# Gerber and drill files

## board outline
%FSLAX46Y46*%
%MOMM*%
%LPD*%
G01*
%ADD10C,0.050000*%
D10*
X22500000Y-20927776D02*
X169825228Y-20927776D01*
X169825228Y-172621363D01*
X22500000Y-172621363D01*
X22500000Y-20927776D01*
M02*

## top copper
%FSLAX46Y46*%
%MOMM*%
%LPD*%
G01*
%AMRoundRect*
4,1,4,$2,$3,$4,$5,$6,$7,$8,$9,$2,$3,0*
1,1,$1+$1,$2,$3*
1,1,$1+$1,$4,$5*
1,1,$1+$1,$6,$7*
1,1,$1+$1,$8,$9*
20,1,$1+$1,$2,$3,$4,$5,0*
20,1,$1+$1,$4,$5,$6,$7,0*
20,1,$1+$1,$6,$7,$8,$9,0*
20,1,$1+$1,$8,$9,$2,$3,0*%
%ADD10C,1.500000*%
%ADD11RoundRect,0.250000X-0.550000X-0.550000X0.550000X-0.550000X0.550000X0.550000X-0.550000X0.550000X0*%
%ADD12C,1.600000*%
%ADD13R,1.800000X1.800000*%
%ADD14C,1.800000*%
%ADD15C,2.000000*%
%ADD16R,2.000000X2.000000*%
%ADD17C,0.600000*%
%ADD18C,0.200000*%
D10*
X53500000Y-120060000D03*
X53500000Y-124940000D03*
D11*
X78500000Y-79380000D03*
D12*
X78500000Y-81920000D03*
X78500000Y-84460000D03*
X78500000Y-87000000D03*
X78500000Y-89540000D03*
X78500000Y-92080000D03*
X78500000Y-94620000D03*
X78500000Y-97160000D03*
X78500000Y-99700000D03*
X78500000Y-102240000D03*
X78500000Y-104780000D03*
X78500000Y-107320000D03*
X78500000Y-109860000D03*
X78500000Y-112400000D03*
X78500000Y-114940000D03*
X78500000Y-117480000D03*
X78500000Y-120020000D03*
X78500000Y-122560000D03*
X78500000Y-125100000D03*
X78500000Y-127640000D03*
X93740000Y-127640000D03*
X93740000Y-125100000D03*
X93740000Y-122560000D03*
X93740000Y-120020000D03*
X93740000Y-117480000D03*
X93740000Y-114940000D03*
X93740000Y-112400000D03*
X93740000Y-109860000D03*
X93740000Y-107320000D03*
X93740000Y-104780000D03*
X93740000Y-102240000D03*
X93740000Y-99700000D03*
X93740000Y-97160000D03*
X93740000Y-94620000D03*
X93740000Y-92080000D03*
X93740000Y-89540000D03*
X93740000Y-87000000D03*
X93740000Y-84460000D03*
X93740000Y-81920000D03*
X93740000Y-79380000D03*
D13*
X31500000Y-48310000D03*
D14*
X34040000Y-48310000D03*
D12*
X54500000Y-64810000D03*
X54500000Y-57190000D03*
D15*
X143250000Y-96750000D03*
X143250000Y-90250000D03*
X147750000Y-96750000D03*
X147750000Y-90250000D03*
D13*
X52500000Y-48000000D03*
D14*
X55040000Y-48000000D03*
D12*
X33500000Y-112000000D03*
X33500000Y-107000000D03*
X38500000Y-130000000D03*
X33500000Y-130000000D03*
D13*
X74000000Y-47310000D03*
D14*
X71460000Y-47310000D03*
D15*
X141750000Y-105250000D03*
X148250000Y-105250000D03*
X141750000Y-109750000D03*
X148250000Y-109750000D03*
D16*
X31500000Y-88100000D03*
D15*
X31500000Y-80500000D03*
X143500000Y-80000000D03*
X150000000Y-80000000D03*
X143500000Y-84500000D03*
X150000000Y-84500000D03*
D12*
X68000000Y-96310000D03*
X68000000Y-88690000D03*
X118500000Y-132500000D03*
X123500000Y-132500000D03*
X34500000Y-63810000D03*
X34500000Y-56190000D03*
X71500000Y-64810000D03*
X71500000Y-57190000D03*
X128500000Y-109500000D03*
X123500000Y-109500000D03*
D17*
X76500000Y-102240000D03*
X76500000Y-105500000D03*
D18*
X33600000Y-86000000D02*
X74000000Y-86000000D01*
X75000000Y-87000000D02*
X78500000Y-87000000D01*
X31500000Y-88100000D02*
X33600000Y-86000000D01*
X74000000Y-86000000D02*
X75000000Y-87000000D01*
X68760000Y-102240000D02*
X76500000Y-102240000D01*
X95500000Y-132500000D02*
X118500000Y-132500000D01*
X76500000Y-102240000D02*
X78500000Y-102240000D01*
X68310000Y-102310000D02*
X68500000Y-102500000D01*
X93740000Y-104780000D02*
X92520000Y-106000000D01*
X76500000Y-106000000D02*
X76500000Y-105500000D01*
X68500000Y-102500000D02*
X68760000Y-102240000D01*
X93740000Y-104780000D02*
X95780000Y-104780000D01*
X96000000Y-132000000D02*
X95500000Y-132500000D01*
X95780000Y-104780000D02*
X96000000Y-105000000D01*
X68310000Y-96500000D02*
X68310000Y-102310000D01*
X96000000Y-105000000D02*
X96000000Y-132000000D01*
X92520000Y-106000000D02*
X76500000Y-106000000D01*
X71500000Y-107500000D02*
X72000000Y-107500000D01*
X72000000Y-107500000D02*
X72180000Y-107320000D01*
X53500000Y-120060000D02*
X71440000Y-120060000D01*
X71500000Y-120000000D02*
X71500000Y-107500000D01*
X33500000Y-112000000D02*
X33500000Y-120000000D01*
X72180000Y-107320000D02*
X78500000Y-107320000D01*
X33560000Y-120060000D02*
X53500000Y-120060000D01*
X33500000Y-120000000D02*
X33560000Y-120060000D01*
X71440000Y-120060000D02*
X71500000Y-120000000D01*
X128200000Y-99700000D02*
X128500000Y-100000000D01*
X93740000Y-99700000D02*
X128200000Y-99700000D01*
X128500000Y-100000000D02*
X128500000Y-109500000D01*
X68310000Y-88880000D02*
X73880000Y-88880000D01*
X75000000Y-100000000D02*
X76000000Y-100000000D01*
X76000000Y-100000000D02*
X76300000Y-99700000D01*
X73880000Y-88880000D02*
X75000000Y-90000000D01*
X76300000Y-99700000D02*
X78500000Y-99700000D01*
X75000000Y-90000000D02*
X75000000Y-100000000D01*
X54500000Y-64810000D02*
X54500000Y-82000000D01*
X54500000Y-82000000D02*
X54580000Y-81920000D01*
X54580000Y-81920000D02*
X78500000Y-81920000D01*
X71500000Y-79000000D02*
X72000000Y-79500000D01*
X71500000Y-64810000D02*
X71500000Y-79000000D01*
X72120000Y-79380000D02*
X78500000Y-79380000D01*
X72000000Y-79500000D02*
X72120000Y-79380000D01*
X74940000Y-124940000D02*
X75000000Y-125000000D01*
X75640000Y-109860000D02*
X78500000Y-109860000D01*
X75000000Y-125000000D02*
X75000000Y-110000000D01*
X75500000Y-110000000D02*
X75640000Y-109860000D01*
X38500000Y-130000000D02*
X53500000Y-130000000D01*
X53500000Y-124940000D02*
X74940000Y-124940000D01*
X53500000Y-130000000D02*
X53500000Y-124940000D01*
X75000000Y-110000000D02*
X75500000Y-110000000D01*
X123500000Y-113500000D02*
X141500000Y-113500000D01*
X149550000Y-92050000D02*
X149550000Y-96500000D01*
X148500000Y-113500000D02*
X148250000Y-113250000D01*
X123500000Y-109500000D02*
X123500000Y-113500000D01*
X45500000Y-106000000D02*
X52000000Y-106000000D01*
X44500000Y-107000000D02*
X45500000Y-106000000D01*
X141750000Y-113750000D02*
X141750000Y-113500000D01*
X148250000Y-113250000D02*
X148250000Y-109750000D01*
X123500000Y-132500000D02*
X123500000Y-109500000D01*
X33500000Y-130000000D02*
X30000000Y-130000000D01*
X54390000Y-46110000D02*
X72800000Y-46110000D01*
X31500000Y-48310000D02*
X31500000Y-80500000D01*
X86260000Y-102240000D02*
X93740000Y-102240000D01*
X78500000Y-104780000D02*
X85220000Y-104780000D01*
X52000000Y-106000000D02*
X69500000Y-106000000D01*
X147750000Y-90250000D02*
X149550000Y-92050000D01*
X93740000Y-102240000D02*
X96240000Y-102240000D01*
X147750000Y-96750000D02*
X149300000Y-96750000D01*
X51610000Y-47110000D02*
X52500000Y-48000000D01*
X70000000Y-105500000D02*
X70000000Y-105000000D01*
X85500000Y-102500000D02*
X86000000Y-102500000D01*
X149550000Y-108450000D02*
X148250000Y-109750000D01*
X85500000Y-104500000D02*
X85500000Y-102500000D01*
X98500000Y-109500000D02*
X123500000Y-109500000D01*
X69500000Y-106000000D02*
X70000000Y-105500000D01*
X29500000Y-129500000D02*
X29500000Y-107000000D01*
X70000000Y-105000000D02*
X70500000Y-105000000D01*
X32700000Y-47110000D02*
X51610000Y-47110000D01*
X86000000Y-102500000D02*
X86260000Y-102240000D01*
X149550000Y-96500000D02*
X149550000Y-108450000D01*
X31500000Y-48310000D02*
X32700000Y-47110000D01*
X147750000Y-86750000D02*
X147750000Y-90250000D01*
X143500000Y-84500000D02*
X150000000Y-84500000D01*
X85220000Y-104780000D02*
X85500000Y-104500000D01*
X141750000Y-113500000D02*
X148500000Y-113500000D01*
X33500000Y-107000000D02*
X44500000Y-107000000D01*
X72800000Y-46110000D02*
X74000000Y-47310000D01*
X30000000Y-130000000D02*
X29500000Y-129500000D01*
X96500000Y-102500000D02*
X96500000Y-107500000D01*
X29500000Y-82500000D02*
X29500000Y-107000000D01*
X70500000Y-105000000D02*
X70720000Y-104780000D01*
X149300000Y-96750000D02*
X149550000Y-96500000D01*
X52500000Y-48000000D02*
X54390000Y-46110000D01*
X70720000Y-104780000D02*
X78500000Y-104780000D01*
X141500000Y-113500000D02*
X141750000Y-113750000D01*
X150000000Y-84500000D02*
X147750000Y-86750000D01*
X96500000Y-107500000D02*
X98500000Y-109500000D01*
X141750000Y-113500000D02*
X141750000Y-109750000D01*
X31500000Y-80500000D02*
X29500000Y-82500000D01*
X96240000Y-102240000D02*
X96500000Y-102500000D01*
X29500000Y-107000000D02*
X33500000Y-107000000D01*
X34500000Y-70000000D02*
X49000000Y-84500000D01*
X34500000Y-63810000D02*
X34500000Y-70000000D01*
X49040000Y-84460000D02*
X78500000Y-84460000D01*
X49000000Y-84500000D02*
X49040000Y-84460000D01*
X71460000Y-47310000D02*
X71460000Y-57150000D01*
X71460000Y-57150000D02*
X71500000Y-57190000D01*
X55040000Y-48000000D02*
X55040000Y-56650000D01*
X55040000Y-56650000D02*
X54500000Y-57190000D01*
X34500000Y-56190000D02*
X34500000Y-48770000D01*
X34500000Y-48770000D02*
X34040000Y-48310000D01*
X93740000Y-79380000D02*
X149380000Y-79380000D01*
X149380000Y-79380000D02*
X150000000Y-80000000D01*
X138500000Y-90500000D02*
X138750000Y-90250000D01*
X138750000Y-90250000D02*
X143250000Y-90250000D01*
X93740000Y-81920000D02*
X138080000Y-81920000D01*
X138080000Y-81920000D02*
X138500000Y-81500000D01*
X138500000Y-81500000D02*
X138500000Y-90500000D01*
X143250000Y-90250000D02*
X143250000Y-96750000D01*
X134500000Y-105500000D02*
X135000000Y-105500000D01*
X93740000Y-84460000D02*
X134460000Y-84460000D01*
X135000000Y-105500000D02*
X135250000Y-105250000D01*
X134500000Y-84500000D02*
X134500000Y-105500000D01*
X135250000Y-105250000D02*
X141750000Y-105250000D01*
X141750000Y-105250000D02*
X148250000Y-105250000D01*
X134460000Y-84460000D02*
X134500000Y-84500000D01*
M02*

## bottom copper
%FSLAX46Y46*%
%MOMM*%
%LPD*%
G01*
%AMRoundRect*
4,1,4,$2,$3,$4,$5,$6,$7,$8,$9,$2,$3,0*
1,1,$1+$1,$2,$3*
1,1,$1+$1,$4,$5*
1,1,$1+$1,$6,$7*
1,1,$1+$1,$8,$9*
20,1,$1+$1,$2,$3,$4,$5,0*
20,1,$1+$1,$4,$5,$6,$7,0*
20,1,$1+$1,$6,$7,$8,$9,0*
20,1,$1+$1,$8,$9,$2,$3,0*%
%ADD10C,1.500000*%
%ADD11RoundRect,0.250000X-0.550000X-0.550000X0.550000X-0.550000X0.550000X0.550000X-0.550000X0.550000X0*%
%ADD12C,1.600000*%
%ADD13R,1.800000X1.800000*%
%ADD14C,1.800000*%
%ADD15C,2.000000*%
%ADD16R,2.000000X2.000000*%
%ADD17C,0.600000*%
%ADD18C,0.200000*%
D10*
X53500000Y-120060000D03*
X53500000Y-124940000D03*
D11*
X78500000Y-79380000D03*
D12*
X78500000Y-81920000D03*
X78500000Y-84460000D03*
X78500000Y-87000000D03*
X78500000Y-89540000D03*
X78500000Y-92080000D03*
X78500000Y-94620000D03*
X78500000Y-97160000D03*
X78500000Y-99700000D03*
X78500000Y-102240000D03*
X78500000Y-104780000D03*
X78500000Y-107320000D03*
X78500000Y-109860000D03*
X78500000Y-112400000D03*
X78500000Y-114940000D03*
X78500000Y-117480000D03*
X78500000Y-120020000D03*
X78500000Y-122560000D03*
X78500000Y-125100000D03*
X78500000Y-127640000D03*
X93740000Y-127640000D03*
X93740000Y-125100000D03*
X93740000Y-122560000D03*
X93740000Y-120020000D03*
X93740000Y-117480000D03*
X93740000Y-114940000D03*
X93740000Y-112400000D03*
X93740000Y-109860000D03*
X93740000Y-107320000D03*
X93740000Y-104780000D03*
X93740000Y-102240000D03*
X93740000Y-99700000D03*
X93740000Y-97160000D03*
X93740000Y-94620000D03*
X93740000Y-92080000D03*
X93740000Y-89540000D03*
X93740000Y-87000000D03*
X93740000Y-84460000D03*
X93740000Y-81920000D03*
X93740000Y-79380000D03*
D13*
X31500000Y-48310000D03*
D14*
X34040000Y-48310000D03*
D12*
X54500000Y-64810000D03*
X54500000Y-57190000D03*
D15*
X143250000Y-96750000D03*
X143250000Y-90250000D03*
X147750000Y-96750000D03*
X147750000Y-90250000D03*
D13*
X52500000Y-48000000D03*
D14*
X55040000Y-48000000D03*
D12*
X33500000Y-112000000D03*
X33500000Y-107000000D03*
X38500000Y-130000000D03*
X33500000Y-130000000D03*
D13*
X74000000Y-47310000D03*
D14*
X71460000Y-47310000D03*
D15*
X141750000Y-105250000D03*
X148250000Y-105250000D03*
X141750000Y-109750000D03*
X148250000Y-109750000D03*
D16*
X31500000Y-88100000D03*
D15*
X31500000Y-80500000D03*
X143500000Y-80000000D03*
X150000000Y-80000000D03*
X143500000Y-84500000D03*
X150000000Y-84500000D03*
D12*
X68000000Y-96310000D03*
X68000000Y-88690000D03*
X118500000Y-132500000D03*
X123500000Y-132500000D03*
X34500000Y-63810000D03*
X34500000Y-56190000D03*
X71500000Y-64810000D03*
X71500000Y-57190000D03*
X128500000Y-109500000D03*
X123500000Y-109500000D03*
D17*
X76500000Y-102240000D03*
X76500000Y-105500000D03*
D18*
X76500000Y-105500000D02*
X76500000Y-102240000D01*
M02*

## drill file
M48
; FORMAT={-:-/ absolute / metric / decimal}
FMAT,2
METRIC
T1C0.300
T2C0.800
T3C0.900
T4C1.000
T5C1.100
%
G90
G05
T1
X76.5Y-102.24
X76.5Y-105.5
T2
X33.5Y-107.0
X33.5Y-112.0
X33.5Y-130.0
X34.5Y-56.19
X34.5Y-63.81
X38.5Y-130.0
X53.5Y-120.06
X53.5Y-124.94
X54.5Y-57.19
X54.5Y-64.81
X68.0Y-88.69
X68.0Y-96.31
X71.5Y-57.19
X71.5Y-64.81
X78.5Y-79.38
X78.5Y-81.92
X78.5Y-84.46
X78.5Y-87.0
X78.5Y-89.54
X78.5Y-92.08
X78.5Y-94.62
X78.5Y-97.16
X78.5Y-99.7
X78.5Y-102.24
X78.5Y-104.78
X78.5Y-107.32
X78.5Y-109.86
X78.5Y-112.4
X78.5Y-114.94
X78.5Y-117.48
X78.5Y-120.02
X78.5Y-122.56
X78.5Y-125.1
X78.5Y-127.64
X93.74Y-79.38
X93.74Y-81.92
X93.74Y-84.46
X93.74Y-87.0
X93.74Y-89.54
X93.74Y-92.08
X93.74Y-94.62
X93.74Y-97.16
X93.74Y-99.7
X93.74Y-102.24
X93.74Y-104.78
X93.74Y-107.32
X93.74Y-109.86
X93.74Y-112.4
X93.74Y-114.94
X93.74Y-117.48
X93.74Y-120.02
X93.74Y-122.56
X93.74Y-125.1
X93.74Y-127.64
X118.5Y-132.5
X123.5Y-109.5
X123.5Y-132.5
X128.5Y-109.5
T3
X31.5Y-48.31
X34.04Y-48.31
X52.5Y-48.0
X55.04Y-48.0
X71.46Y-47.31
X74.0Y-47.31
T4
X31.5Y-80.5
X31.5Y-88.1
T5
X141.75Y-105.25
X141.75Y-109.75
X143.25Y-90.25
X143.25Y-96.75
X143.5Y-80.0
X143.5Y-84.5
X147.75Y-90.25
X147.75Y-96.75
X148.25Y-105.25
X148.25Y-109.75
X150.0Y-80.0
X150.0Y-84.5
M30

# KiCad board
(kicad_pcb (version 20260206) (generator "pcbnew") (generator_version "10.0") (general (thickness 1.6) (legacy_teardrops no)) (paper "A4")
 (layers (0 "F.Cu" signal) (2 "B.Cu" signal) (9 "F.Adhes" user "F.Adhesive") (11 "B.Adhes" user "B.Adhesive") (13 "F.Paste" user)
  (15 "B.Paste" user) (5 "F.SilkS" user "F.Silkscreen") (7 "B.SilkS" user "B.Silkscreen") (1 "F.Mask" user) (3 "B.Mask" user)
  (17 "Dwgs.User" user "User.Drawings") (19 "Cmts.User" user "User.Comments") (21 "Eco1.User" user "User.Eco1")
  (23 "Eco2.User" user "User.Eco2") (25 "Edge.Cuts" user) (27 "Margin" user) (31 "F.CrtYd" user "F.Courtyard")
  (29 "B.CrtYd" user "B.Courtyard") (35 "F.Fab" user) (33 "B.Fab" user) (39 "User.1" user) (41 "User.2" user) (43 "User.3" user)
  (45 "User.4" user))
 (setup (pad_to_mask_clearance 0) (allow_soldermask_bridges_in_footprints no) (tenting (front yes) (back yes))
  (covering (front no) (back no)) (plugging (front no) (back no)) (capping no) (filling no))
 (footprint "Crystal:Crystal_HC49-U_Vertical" (layer "F.Cu") (at 53.5 120.06 -90)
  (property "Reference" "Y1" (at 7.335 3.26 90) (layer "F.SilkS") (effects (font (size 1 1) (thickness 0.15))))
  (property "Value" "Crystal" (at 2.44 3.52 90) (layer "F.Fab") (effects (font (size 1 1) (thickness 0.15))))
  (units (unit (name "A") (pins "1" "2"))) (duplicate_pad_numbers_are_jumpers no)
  (pad "1" thru_hole circle (at 0 0 270) (size 1.5 1.5) (drill 0.8) (layers "*.Cu" "*.Mask") (remove_unused_layers no)
   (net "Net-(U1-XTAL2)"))
  (pad "2" thru_hole circle (at 4.88 0 270) (size 1.5 1.5) (drill 0.8) (layers "*.Cu" "*.Mask") (remove_unused_layers no)
   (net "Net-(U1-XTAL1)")))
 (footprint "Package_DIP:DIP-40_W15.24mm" (layer "F.Cu") (at 78.5 79.38)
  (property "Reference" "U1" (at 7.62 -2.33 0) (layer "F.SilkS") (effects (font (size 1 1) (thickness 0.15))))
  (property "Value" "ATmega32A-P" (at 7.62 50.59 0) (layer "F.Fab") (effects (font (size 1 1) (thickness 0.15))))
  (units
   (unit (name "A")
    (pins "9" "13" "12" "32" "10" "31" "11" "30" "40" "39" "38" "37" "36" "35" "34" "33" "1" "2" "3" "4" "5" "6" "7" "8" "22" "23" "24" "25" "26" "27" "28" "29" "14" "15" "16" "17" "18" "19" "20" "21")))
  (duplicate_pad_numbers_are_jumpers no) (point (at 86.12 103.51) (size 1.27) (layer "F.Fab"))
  (pad "1" thru_hole roundrect (at 0 0) (size 1.6 1.6) (drill 0.8) (layers "*.Cu" "*.Mask") (remove_unused_layers no)
   (roundrect_rratio 0.15625) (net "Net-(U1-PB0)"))
  (pad "2" thru_hole circle (at 0 2.54) (size 1.6 1.6) (drill 0.8) (layers "*.Cu" "*.Mask") (remove_unused_layers no) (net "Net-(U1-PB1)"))
  (pad "3" thru_hole circle (at 0 5.08) (size 1.6 1.6) (drill 0.8) (layers "*.Cu" "*.Mask") (remove_unused_layers no) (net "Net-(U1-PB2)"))
  (pad "4" thru_hole circle (at 0 7.62) (size 1.6 1.6) (drill 0.8) (layers "*.Cu" "*.Mask") (remove_unused_layers no) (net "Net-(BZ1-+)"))
  (pad "5" thru_hole circle (at 0 10.16) (size 1.6 1.6) (drill 0.8) (layers "*.Cu" "*.Mask") (remove_unused_layers no)
   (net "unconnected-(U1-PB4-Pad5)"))
  (pad "6" thru_hole circle (at 0 12.7) (size 1.6 1.6) (drill 0.8) (layers "*.Cu" "*.Mask") (remove_unused_layers no)
   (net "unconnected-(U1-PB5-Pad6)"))
  (pad "7" thru_hole circle (at 0 15.24) (size 1.6 1.6) (drill 0.8) (layers "*.Cu" "*.Mask") (remove_unused_layers no)
   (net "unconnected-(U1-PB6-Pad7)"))
  (pad "8" thru_hole circle (at 0 17.78) (size 1.6 1.6) (drill 0.8) (layers "*.Cu" "*.Mask") (remove_unused_layers no)
   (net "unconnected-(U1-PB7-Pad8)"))
  (pad "9" thru_hole circle (at 0 20.32) (size 1.6 1.6) (drill 0.8) (layers "*.Cu" "*.Mask") (remove_unused_layers no)
   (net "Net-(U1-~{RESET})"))
  (pad "10" thru_hole circle (at 0 22.86) (size 1.6 1.6) (drill 0.8) (layers "*.Cu" "*.Mask") (remove_unused_layers no) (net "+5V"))
  (pad "11" thru_hole circle (at 0 25.4) (size 1.6 1.6) (drill 0.8) (layers "*.Cu" "*.Mask") (remove_unused_layers no) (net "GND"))
  (pad "12" thru_hole circle (at 0 27.94) (size 1.6 1.6) (drill 0.8) (layers "*.Cu" "*.Mask") (remove_unused_layers no)
   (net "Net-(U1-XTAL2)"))
  (pad "13" thru_hole circle (at 0 30.48) (size 1.6 1.6) (drill 0.8) (layers "*.Cu" "*.Mask") (remove_unused_layers no)
   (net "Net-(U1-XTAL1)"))
  (pad "14" thru_hole circle (at 0 33.02) (size 1.6 1.6) (drill 0.8) (layers "*.Cu" "*.Mask") (remove_unused_layers no)
   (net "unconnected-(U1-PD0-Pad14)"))
  (pad "15" thru_hole circle (at 0 35.56) (size 1.6 1.6) (drill 0.8) (layers "*.Cu" "*.Mask") (remove_unused_layers no)
   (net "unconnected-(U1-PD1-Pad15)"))
  (pad "16" thru_hole circle (at 0 38.1) (size 1.6 1.6) (drill 0.8) (layers "*.Cu" "*.Mask") (remove_unused_layers no)
   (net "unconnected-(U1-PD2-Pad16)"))
  (pad "17" thru_hole circle (at 0 40.64) (size 1.6 1.6) (drill 0.8) (layers "*.Cu" "*.Mask") (remove_unused_layers no)
   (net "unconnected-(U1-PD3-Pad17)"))
  (pad "18" thru_hole circle (at 0 43.18) (size 1.6 1.6) (drill 0.8) (layers "*.Cu" "*.Mask") (remove_unused_layers no)
   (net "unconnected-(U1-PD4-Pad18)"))
  (pad "19" thru_hole circle (at 0 45.72) (size 1.6 1.6) (drill 0.8) (layers "*.Cu" "*.Mask") (remove_unused_layers no)
   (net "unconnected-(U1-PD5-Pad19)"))
  (pad "20" thru_hole circle (at 0 48.26) (size 1.6 1.6) (drill 0.8) (layers "*.Cu" "*.Mask") (remove_unused_layers no)
   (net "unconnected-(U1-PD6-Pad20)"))
  (pad "21" thru_hole circle (at 15.24 48.26) (size 1.6 1.6) (drill 0.8) (layers "*.Cu" "*.Mask") (remove_unused_layers no)
   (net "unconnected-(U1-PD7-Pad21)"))
  (pad "22" thru_hole circle (at 15.24 45.72) (size 1.6 1.6) (drill 0.8) (layers "*.Cu" "*.Mask") (remove_unused_layers no)
   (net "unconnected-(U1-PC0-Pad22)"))
  (pad "23" thru_hole circle (at 15.24 43.18) (size 1.6 1.6) (drill 0.8) (layers "*.Cu" "*.Mask") (remove_unused_layers no)
   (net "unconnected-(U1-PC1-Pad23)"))
  (pad "24" thru_hole circle (at 15.24 40.64) (size 1.6 1.6) (drill 0.8) (layers "*.Cu" "*.Mask") (remove_unused_layers no)
   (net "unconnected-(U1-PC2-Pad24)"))
  (pad "25" thru_hole circle (at 15.24 38.1) (size 1.6 1.6) (drill 0.8) (layers "*.Cu" "*.Mask") (remove_unused_layers no)
   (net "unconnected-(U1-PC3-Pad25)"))
  (pad "26" thru_hole circle (at 15.24 35.56) (size 1.6 1.6) (drill 0.8) (layers "*.Cu" "*.Mask") (remove_unused_layers no)
   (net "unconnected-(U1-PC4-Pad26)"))
  (pad "27" thru_hole circle (at 15.24 33.02) (size 1.6 1.6) (drill 0.8) (layers "*.Cu" "*.Mask") (remove_unused_layers no)
   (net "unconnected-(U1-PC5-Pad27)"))
  (pad "28" thru_hole circle (at 15.24 30.48) (size 1.6 1.6) (drill 0.8) (layers "*.Cu" "*.Mask") (remove_unused_layers no)
   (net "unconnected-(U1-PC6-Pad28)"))
  (pad "29" thru_hole circle (at 15.24 27.94) (size 1.6 1.6) (drill 0.8) (layers "*.Cu" "*.Mask") (remove_unused_layers no)
   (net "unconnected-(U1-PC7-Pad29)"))
  (pad "30" thru_hole circle (at 15.24 25.4) (size 1.6 1.6) (drill 0.8) (layers "*.Cu" "*.Mask") (remove_unused_layers no) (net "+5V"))
  (pad "31" thru_hole circle (at 15.24 22.86) (size 1.6 1.6) (drill 0.8) (layers "*.Cu" "*.Mask") (remove_unused_layers no) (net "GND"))
  (pad "32" thru_hole circle (at 15.24 20.32) (size 1.6 1.6) (drill 0.8) (layers "*.Cu" "*.Mask") (remove_unused_layers no)
   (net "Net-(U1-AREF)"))
  (pad "33" thru_hole circle (at 15.24 17.78) (size 1.6 1.6) (drill 0.8) (layers "*.Cu" "*.Mask") (remove_unused_layers no)
   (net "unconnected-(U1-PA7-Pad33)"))
  (pad "34" thru_hole circle (at 15.24 15.24) (size 1.6 1.6) (drill 0.8) (layers "*.Cu" "*.Mask") (remove_unused_layers no)
   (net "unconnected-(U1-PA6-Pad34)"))
  (pad "35" thru_hole circle (at 15.24 12.7) (size 1.6 1.6) (drill 0.8) (layers "*.Cu" "*.Mask") (remove_unused_layers no)
   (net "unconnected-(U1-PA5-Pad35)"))
  (pad "36" thru_hole circle (at 15.24 10.16) (size 1.6 1.6) (drill 0.8) (layers "*.Cu" "*.Mask") (remove_unused_layers no)
   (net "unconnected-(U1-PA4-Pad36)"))
  (pad "37" thru_hole circle (at 15.24 7.62) (size 1.6 1.6) (drill 0.8) (layers "*.Cu" "*.Mask") (remove_unused_layers no)
   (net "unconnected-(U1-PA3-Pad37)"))
  (pad "38" thru_hole circle (at 15.24 5.08) (size 1.6 1.6) (drill 0.8) (layers "*.Cu" "*.Mask") (remove_unused_layers no)
   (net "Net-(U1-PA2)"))
  (pad "39" thru_hole circle (at 15.24 2.54) (size 1.6 1.6) (drill 0.8) (layers "*.Cu" "*.Mask") (remove_unused_layers no)
   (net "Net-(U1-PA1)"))
  (pad "40" thru_hole circle (at 15.24 0) (size 1.6 1.6) (drill 0.8) (layers "*.Cu" "*.Mask") (remove_unused_layers no) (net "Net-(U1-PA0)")))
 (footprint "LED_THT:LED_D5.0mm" (layer "F.Cu") (at 31.5 48.31)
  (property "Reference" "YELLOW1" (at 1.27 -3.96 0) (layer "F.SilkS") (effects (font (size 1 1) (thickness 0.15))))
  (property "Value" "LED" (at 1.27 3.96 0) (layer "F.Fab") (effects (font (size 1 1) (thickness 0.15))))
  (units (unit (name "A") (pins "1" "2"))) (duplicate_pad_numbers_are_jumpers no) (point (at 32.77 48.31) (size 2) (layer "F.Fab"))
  (pad "1" thru_hole rect (at 0 0) (size 1.8 1.8) (drill 0.9) (layers "*.Cu" "*.Mask") (remove_unused_layers no) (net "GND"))
  (pad "2" thru_hole circle (at 2.54 0) (size 1.8 1.8) (drill 0.9) (layers "*.Cu" "*.Mask") (remove_unused_layers no)
   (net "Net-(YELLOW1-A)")))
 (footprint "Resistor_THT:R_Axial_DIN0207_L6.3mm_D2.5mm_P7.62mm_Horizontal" (layer "F.Cu") (at 54.5 64.81 90)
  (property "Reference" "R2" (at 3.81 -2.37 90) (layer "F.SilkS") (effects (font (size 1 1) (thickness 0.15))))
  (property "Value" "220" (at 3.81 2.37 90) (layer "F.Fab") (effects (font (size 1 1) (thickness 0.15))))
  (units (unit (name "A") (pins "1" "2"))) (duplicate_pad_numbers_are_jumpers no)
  (pad "1" thru_hole circle (at 0 0 90) (size 1.6 1.6) (drill 0.8) (layers "*.Cu" "*.Mask") (remove_unused_layers no) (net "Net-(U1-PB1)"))
  (pad "2" thru_hole circle (at 7.62 0 90) (size 1.6 1.6) (drill 0.8) (layers "*.Cu" "*.Mask") (remove_unused_layers no)
   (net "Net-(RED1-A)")))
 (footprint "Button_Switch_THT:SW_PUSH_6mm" (layer "F.Cu") (at 143.25 96.75 90)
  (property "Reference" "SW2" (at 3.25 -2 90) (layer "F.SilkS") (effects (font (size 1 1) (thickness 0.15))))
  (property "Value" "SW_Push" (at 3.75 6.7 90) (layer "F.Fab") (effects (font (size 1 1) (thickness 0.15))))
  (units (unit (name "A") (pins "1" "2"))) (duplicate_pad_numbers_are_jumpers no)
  (pad "1" thru_hole circle (at 0 0 180) (size 2 2) (drill 1.1) (layers "*.Cu" "*.Mask") (remove_unused_layers no) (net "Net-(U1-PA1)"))
  (pad "1" thru_hole circle (at 6.5 0 180) (size 2 2) (drill 1.1) (layers "*.Cu" "*.Mask") (remove_unused_layers no) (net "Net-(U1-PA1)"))
  (pad "2" thru_hole circle (at 0 4.5 180) (size 2 2) (drill 1.1) (layers "*.Cu" "*.Mask") (remove_unused_layers no) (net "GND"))
  (pad "2" thru_hole circle (at 6.5 4.5 180) (size 2 2) (drill 1.1) (layers "*.Cu" "*.Mask") (remove_unused_layers no) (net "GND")))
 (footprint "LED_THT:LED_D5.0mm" (layer "F.Cu") (at 52.5 48)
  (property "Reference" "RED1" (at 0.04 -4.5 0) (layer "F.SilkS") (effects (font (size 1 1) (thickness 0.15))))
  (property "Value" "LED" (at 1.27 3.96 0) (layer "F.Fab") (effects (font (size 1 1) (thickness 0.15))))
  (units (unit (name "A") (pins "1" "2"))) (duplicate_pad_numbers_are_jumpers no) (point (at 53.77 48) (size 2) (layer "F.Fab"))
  (pad "1" thru_hole rect (at 0 0) (size 1.8 1.8) (drill 0.9) (layers "*.Cu" "*.Mask") (remove_unused_layers no) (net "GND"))
  (pad "2" thru_hole circle (at 2.54 0) (size 1.8 1.8) (drill 0.9) (layers "*.Cu" "*.Mask") (remove_unused_layers no) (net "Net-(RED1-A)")))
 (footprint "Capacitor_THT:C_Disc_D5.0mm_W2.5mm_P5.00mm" (layer "F.Cu") (at 33.5 112 90)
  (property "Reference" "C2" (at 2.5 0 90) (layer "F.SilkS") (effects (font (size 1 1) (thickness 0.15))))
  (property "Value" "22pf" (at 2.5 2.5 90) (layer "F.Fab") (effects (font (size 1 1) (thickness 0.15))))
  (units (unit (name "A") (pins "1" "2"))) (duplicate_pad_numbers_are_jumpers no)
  (pad "1" thru_hole circle (at 0 0 90) (size 1.6 1.6) (drill 0.8) (layers "*.Cu" "*.Mask") (remove_unused_layers no) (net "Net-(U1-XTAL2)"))
  (pad "2" thru_hole circle (at 5 0 90) (size 1.6 1.6) (drill 0.8) (layers "*.Cu" "*.Mask") (remove_unused_layers no) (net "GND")))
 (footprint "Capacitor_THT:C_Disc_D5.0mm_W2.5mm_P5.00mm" (layer "F.Cu") (at 38.5 130 180)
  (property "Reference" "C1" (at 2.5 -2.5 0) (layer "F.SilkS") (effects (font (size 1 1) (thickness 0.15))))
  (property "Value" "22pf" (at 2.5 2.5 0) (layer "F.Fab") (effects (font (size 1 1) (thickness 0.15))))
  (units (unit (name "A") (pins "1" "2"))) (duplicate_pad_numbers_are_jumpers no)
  (pad "1" thru_hole circle (at 0 0 180) (size 1.6 1.6) (drill 0.8) (layers "*.Cu" "*.Mask") (remove_unused_layers no)
   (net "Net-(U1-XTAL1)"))
  (pad "2" thru_hole circle (at 5 0 180) (size 1.6 1.6) (drill 0.8) (layers "*.Cu" "*.Mask") (remove_unused_layers no) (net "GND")))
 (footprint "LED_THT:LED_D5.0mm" (layer "F.Cu") (at 74 47.31 180)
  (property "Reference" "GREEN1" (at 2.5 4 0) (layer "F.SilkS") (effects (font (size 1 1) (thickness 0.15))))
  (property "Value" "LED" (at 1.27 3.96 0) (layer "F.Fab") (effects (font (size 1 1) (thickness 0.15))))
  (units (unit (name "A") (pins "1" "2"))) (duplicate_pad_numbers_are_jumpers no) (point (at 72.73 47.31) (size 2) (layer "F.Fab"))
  (pad "1" thru_hole rect (at 0 0 180) (size 1.8 1.8) (drill 0.9) (layers "*.Cu" "*.Mask") (remove_unused_layers no) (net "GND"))
  (pad "2" thru_hole circle (at 2.54 0 180) (size 1.8 1.8) (drill 0.9) (layers "*.Cu" "*.Mask") (remove_unused_layers no)
   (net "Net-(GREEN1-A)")))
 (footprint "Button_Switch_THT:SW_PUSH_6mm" (layer "F.Cu") (at 141.75 105.25)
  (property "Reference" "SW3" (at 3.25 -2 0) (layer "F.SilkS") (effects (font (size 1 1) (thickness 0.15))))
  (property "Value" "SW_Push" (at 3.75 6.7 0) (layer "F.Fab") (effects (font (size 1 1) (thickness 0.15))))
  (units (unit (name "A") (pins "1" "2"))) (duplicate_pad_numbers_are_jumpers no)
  (pad "1" thru_hole circle (at 0 0 90) (size 2 2) (drill 1.1) (layers "*.Cu" "*.Mask") (remove_unused_layers no) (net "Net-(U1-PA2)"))
  (pad "1" thru_hole circle (at 6.5 0 90) (size 2 2) (drill 1.1) (layers "*.Cu" "*.Mask") (remove_unused_layers no) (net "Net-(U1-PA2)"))
  (pad "2" thru_hole circle (at 0 4.5 90) (size 2 2) (drill 1.1) (layers "*.Cu" "*.Mask") (remove_unused_layers no) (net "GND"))
  (pad "2" thru_hole circle (at 6.5 4.5 90) (size 2 2) (drill 1.1) (layers "*.Cu" "*.Mask") (remove_unused_layers no) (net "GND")))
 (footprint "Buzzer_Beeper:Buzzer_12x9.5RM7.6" (layer "F.Cu") (at 31.5 88.1 90)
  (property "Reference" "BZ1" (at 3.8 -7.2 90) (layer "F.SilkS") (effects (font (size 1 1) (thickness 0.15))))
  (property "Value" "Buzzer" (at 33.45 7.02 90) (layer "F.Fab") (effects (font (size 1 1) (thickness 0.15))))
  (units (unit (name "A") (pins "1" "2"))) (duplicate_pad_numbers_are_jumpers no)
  (pad "1" thru_hole rect (at 0 0 90) (size 2 2) (drill 1) (layers "*.Cu" "*.Mask") (remove_unused_layers no) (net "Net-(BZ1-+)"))
  (pad "2" thru_hole circle (at 7.6 0 90) (size 2 2) (drill 1) (layers "*.Cu" "*.Mask") (remove_unused_layers no) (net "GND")))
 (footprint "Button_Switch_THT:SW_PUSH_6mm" (layer "F.Cu") (at 143.5 80)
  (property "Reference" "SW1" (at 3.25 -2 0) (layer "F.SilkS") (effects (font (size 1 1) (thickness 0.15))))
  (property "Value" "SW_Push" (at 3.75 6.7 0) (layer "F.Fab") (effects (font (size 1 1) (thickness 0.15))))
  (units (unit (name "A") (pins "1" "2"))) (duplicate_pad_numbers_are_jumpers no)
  (pad "1" thru_hole circle (at 0 0 90) (size 2 2) (drill 1.1) (layers "*.Cu" "*.Mask") (remove_unused_layers no) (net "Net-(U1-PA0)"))
  (pad "1" thru_hole circle (at 6.5 0 90) (size 2 2) (drill 1.1) (layers "*.Cu" "*.Mask") (remove_unused_layers no) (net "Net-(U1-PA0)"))
  (pad "2" thru_hole circle (at 0 4.5 90) (size 2 2) (drill 1.1) (layers "*.Cu" "*.Mask") (remove_unused_layers no) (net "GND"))
  (pad "2" thru_hole circle (at 6.5 4.5 90) (size 2 2) (drill 1.1) (layers "*.Cu" "*.Mask") (remove_unused_layers no) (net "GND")))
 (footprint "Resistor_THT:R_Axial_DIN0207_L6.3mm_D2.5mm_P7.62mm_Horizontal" (layer "F.Cu") (at 68 96.31 90)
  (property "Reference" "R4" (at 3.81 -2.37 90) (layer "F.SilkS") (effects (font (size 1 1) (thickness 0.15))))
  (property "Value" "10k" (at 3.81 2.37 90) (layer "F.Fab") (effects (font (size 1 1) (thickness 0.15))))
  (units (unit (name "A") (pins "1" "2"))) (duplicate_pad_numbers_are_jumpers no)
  (pad "1" thru_hole circle (at 0 0 90) (size 1.6 1.6) (drill 0.8) (layers "*.Cu" "*.Mask") (remove_unused_layers no) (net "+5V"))
  (pad "2" thru_hole circle (at 7.62 0 90) (size 1.6 1.6) (drill 0.8) (layers "*.Cu" "*.Mask") (remove_unused_layers no)
   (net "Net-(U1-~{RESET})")))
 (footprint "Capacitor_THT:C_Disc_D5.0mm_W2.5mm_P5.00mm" (layer "F.Cu") (at 118.5 132.5)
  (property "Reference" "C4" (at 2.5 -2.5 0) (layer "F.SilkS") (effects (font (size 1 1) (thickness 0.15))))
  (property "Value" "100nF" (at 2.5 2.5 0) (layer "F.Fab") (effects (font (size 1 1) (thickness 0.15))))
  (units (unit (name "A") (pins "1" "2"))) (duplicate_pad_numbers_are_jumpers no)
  (pad "1" thru_hole circle (at 0 0) (size 1.6 1.6) (drill 0.8) (layers "*.Cu" "*.Mask") (remove_unused_layers no) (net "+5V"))
  (pad "2" thru_hole circle (at 5 0) (size 1.6 1.6) (drill 0.8) (layers "*.Cu" "*.Mask") (remove_unused_layers no) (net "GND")))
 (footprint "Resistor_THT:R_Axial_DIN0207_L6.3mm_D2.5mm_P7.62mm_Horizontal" (layer "F.Cu") (at 34.5 63.81 90)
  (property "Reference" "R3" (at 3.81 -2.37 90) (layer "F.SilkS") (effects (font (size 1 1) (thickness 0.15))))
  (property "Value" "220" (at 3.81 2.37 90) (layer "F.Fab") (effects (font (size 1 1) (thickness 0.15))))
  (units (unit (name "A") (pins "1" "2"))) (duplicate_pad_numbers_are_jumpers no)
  (pad "1" thru_hole circle (at 0 0 90) (size 1.6 1.6) (drill 0.8) (layers "*.Cu" "*.Mask") (remove_unused_layers no) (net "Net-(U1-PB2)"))
  (pad "2" thru_hole circle (at 7.62 0 90) (size 1.6 1.6) (drill 0.8) (layers "*.Cu" "*.Mask") (remove_unused_layers no)
   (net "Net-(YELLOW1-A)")))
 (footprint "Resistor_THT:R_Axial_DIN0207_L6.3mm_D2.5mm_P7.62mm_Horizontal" (layer "F.Cu") (at 71.5 64.81 90)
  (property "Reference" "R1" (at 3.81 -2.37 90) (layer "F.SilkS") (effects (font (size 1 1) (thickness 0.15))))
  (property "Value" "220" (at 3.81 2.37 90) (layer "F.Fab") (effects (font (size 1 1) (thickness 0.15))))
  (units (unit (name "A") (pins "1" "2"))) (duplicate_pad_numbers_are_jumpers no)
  (pad "1" thru_hole circle (at 0 0 90) (size 1.6 1.6) (drill 0.8) (layers "*.Cu" "*.Mask") (remove_unused_layers no) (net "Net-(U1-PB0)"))
  (pad "2" thru_hole circle (at 7.62 0 90) (size 1.6 1.6) (drill 0.8) (layers "*.Cu" "*.Mask") (remove_unused_layers no)
   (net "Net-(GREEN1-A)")))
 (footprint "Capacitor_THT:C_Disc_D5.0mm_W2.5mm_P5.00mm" (layer "F.Cu") (at 128.5 109.5 180)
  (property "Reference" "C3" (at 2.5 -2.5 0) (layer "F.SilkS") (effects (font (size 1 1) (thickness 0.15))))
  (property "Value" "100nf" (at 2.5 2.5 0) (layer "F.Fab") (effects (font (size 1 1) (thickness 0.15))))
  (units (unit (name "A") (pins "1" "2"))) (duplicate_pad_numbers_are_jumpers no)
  (pad "1" thru_hole circle (at 0 0 180) (size 1.6 1.6) (drill 0.8) (layers "*.Cu" "*.Mask") (remove_unused_layers no) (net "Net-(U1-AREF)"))
  (pad "2" thru_hole circle (at 5 0 180) (size 1.6 1.6) (drill 0.8) (layers "*.Cu" "*.Mask") (remove_unused_layers no) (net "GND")))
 (gr_rect (start 22.5 20.927776) (end 169.825228 172.621363) (stroke (width 0.05) (type default)) (fill no) (layer "Edge.Cuts"))
 (segment (start 33.6 86) (end 74 86) (width 0.2) (layer "F.Cu") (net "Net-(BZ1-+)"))
 (segment (start 75 87) (end 78.5 87) (width 0.2) (layer "F.Cu") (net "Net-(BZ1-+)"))
 (segment (start 31.5 88.1) (end 33.6 86) (width 0.2) (layer "F.Cu") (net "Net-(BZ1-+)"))
 (segment (start 74 86) (end 75 87) (width 0.2) (layer "F.Cu") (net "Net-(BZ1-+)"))
 (segment (start 68.76 102.24) (end 76.5 102.24) (width 0.2) (layer "F.Cu") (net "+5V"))
 (segment (start 95.5 132.5) (end 118.5 132.5) (width 0.2) (layer "F.Cu") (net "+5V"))
 (segment (start 76.5 102.24) (end 78.5 102.24) (width 0.2) (layer "F.Cu") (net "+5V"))
 (segment (start 68.31 102.31) (end 68.5 102.5) (width 0.2) (layer "F.Cu") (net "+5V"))
 (segment (start 93.74 104.78) (end 92.52 106) (width 0.2) (layer "F.Cu") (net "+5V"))
 (segment (start 76.5 106) (end 76.5 105.5) (width 0.2) (layer "F.Cu") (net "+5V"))
 (segment (start 68.5 102.5) (end 68.76 102.24) (width 0.2) (layer "F.Cu") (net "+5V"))
 (segment (start 93.74 104.78) (end 95.78 104.78) (width 0.2) (layer "F.Cu") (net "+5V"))
 (segment (start 96 132) (end 95.5 132.5) (width 0.2) (layer "F.Cu") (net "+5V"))
 (segment (start 95.78 104.78) (end 96 105) (width 0.2) (layer "F.Cu") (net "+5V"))
 (segment (start 68.31 96.5) (end 68.31 102.31) (width 0.2) (layer "F.Cu") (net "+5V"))
 (segment (start 96 105) (end 96 132) (width 0.2) (layer "F.Cu") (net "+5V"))
 (segment (start 92.52 106) (end 76.5 106) (width 0.2) (layer "F.Cu") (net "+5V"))
 (via (at 76.5 102.24) (size 0.6) (drill 0.3) (layers "F.Cu" "B.Cu") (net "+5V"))
 (via (at 76.5 105.5) (size 0.6) (drill 0.3) (layers "F.Cu" "B.Cu") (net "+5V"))
 (segment (start 76.5 105.5) (end 76.5 102.24) (width 0.2) (layer "B.Cu") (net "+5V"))
 (segment (start 71.5 107.5) (end 72 107.5) (width 0.2) (layer "F.Cu") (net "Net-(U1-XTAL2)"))
 (segment (start 72 107.5) (end 72.18 107.32) (width 0.2) (layer "F.Cu") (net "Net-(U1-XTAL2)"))
 (segment (start 53.5 120.06) (end 71.44 120.06) (width 0.2) (layer "F.Cu") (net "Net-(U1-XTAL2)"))
 (segment (start 71.5 120) (end 71.5 107.5) (width 0.2) (layer "F.Cu") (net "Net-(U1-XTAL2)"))
 (segment (start 33.5 112) (end 33.5 120) (width 0.2) (layer "F.Cu") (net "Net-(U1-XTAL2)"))
 (segment (start 72.18 107.32) (end 78.5 107.32) (width 0.2) (layer "F.Cu") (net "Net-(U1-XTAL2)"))
 (segment (start 33.56 120.06) (end 53.5 120.06) (width 0.2) (layer "F.Cu") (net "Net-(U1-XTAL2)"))
 (segment (start 33.5 120) (end 33.56 120.06) (width 0.2) (layer "F.Cu") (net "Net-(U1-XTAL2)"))
 (segment (start 71.44 120.06) (end 71.5 120) (width 0.2) (layer "F.Cu") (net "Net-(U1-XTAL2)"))
 (segment (start 128.2 99.7) (end 128.5 100) (width 0.2) (layer "F.Cu") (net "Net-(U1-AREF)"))
 (segment (start 93.74 99.7) (end 128.2 99.7) (width 0.2) (layer "F.Cu") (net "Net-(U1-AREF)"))
 (segment (start 128.5 100) (end 128.5 109.5) (width 0.2) (layer "F.Cu") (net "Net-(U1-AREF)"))
 (segment (start 68.31 88.88) (end 73.88 88.88) (width 0.2) (layer "F.Cu") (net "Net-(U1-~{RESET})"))
 (segment (start 75 100) (end 76 100) (width 0.2) (layer "F.Cu") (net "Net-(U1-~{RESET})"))
 (segment (start 76 100) (end 76.3 99.7) (width 0.2) (layer "F.Cu") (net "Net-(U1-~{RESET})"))
 (segment (start 73.88 88.88) (end 75 90) (width 0.2) (layer "F.Cu") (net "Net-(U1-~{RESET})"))
 (segment (start 76.3 99.7) (end 78.5 99.7) (width 0.2) (layer "F.Cu") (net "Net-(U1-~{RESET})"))
 (segment (start 75 90) (end 75 100) (width 0.2) (layer "F.Cu") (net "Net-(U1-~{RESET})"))
 (segment (start 54.5 64.81) (end 54.5 82) (width 0.2) (layer "F.Cu") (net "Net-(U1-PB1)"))
 (segment (start 54.5 82) (end 54.58 81.92) (width 0.2) (layer "F.Cu") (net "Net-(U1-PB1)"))
 (segment (start 54.58 81.92) (end 78.5 81.92) (width 0.2) (layer "F.Cu") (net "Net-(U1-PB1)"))
 (segment (start 71.5 79) (end 72 79.5) (width 0.2) (layer "F.Cu") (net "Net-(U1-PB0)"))
 (segment (start 71.5 64.81) (end 71.5 79) (width 0.2) (layer "F.Cu") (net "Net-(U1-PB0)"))
 (segment (start 72.12 79.38) (end 78.5 79.38) (width 0.2) (layer "F.Cu") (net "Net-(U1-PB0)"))
 (segment (start 72 79.5) (end 72.12 79.38) (width 0.2) (layer "F.Cu") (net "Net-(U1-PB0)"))
 (segment (start 74.94 124.94) (end 75 125) (width 0.2) (layer "F.Cu") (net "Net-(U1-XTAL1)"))
 (segment (start 75.64 109.86) (end 78.5 109.86) (width 0.2) (layer "F.Cu") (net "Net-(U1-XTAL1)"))
 (segment (start 75 125) (end 75 110) (width 0.2) (layer "F.Cu") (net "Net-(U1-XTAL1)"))
 (segment (start 75.5 110) (end 75.64 109.86) (width 0.2) (layer "F.Cu") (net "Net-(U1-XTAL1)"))
 (segment (start 38.5 130) (end 53.5 130) (width 0.2) (layer "F.Cu") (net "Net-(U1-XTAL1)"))
 (segment (start 53.5 124.94) (end 74.94 124.94) (width 0.2) (layer "F.Cu") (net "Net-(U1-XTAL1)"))
 (segment (start 53.5 130) (end 53.5 124.94) (width 0.2) (layer "F.Cu") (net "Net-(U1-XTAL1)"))
 (segment (start 75 110) (end 75.5 110) (width 0.2) (layer "F.Cu") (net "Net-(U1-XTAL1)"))
 (segment (start 123.5 113.5) (end 141.5 113.5) (width 0.2) (layer "F.Cu") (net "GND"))
 (segment (start 149.55 92.05) (end 149.55 96.5) (width 0.2) (layer "F.Cu") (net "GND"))
 (segment (start 148.5 113.5) (end 148.25 113.25) (width 0.2) (layer "F.Cu") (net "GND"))
 (segment (start 123.5 109.5) (end 123.5 113.5) (width 0.2) (layer "F.Cu") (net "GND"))
 (segment (start 45.5 106) (end 52 106) (width 0.2) (layer "F.Cu") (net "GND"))
 (segment (start 44.5 107) (end 45.5 106) (width 0.2) (layer "F.Cu") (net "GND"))
 (segment (start 141.75 113.75) (end 141.75 113.5) (width 0.2) (layer "F.Cu") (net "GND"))
 (segment (start 148.25 113.25) (end 148.25 109.75) (width 0.2) (layer "F.Cu") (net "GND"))
 (segment (start 123.5 132.5) (end 123.5 109.5) (width 0.2) (layer "F.Cu") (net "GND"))
 (segment (start 33.5 130) (end 30 130) (width 0.2) (layer "F.Cu") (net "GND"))
 (segment (start 54.39 46.11) (end 72.8 46.11) (width 0.2) (layer "F.Cu") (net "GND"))
 (segment (start 31.5 48.31) (end 31.5 80.5) (width 0.2) (layer "F.Cu") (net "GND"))
 (segment (start 86.26 102.24) (end 93.74 102.24) (width 0.2) (layer "F.Cu") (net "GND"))
 (segment (start 78.5 104.78) (end 85.22 104.78) (width 0.2) (layer "F.Cu") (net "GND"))
 (segment (start 52 106) (end 69.5 106) (width 0.2) (layer "F.Cu") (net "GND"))
 (segment (start 147.75 90.25) (end 149.55 92.05) (width 0.2) (layer "F.Cu") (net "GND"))
 (segment (start 93.74 102.24) (end 96.24 102.24) (width 0.2) (layer "F.Cu") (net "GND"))
 (segment (start 147.75 96.75) (end 149.3 96.75) (width 0.2) (layer "F.Cu") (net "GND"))
 (segment (start 51.61 47.11) (end 52.5 48) (width 0.2) (layer "F.Cu") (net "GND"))
 (segment (start 70 105.5) (end 70 105) (width 0.2) (layer "F.Cu") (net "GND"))
 (segment (start 85.5 102.5) (end 86 102.5) (width 0.2) (layer "F.Cu") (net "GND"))
 (segment (start 149.55 108.45) (end 148.25 109.75) (width 0.2) (layer "F.Cu") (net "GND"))
 (segment (start 85.5 104.5) (end 85.5 102.5) (width 0.2) (layer "F.Cu") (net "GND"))
 (segment (start 98.5 109.5) (end 123.5 109.5) (width 0.2) (layer "F.Cu") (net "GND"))
 (segment (start 69.5 106) (end 70 105.5) (width 0.2) (layer "F.Cu") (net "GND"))
 (segment (start 29.5 129.5) (end 29.5 107) (width 0.2) (layer "F.Cu") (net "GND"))
 (segment (start 70 105) (end 70.5 105) (width 0.2) (layer "F.Cu") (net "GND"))
 (segment (start 32.7 47.11) (end 51.61 47.11) (width 0.2) (layer "F.Cu") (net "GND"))
 (segment (start 86 102.5) (end 86.26 102.24) (width 0.2) (layer "F.Cu") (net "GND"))
 (segment (start 149.55 96.5) (end 149.55 108.45) (width 0.2) (layer "F.Cu") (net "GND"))
 (segment (start 31.5 48.31) (end 32.7 47.11) (width 0.2) (layer "F.Cu") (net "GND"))
 (segment (start 147.75 86.75) (end 147.75 90.25) (width 0.2) (layer "F.Cu") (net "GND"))
 (segment (start 143.5 84.5) (end 150 84.5) (width 0.2) (layer "F.Cu") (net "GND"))
 (segment (start 85.22 104.78) (end 85.5 104.5) (width 0.2) (layer "F.Cu") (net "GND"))
 (segment (start 141.75 113.5) (end 148.5 113.5) (width 0.2) (layer "F.Cu") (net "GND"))
 (segment (start 33.5 107) (end 44.5 107) (width 0.2) (layer "F.Cu") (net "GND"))
 (segment (start 72.8 46.11) (end 74 47.31) (width 0.2) (layer "F.Cu") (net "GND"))
 (segment (start 30 130) (end 29.5 129.5) (width 0.2) (layer "F.Cu") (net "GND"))
 (segment (start 96.5 102.5) (end 96.5 107.5) (width 0.2) (layer "F.Cu") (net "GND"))
 (segment (start 29.5 82.5) (end 29.5 107) (width 0.2) (layer "F.Cu") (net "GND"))
 (segment (start 70.5 105) (end 70.72 104.78) (width 0.2) (layer "F.Cu") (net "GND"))
 (segment (start 149.3 96.75) (end 149.55 96.5) (width 0.2) (layer "F.Cu") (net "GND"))
 (segment (start 52.5 48) (end 54.39 46.11) (width 0.2) (layer "F.Cu") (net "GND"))
 (segment (start 70.72 104.78) (end 78.5 104.78) (width 0.2) (layer "F.Cu") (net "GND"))
 (segment (start 141.5 113.5) (end 141.75 113.75) (width 0.2) (layer "F.Cu") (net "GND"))
 (segment (start 150 84.5) (end 147.75 86.75) (width 0.2) (layer "F.Cu") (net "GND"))
 (segment (start 96.5 107.5) (end 98.5 109.5) (width 0.2) (layer "F.Cu") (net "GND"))
 (segment (start 141.75 113.5) (end 141.75 109.75) (width 0.2) (layer "F.Cu") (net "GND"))
 (segment (start 31.5 80.5) (end 29.5 82.5) (width 0.2) (layer "F.Cu") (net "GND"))
 (segment (start 96.24 102.24) (end 96.5 102.5) (width 0.2) (layer "F.Cu") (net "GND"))
 (segment (start 29.5 107) (end 33.5 107) (width 0.2) (layer "F.Cu") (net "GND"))
 (segment (start 34.5 70) (end 49 84.5) (width 0.2) (layer "F.Cu") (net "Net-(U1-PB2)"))
 (segment (start 34.5 63.81) (end 34.5 70) (width 0.2) (layer "F.Cu") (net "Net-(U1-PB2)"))
 (segment (start 49.04 84.46) (end 78.5 84.46) (width 0.2) (layer "F.Cu") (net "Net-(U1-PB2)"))
 (segment (start 49 84.5) (end 49.04 84.46) (width 0.2) (layer "F.Cu") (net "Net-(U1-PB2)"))
 (segment (start 71.46 47.31) (end 71.46 57.15) (width 0.2) (layer "F.Cu") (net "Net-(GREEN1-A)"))
 (segment (start 71.46 57.15) (end 71.5 57.19) (width 0.2) (layer "F.Cu") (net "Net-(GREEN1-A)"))
 (segment (start 55.04 48) (end 55.04 56.65) (width 0.2) (layer "F.Cu") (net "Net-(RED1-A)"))
 (segment (start 55.04 56.65) (end 54.5 57.19) (width 0.2) (layer "F.Cu") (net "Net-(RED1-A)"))
 (segment (start 34.5 56.19) (end 34.5 48.77) (width 0.2) (layer "F.Cu") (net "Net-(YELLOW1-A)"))
 (segment (start 34.5 48.77) (end 34.04 48.31) (width 0.2) (layer "F.Cu") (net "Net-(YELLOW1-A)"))
 (segment (start 93.74 79.38) (end 149.38 79.38) (width 0.2) (layer "F.Cu") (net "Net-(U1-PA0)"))
 (segment (start 149.38 79.38) (end 150 80) (width 0.2) (layer "F.Cu") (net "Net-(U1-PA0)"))
 (segment (start 138.5 90.5) (end 138.75 90.25) (width 0.2) (layer "F.Cu") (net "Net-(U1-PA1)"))
 (segment (start 138.75 90.25) (end 143.25 90.25) (width 0.2) (layer "F.Cu") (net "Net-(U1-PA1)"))
 (segment (start 93.74 81.92) (end 138.08 81.92) (width 0.2) (layer "F.Cu") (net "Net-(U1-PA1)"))
 (segment (start 138.08 81.92) (end 138.5 81.5) (width 0.2) (layer "F.Cu") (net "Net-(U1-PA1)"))
 (segment (start 138.5 81.5) (end 138.5 90.5) (width 0.2) (layer "F.Cu") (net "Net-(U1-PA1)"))
 (segment (start 143.25 90.25) (end 143.25 96.75) (width 0.2) (layer "F.Cu") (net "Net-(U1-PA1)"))
 (segment (start 134.5 105.5) (end 135 105.5) (width 0.2) (layer "F.Cu") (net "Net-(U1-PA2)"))
 (segment (start 93.74 84.46) (end 134.46 84.46) (width 0.2) (layer "F.Cu") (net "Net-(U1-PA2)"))
 (segment (start 135 105.5) (end 135.25 105.25) (width 0.2) (layer "F.Cu") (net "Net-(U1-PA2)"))
 (segment (start 134.5 84.5) (end 134.5 105.5) (width 0.2) (layer "F.Cu") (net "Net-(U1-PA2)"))
 (segment (start 135.25 105.25) (end 141.75 105.25) (width 0.2) (layer "F.Cu") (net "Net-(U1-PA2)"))
 (segment (start 141.75 105.25) (end 148.25 105.25) (width 0.2) (layer "F.Cu") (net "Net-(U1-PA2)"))
 (segment (start 134.46 84.46) (end 134.5 84.5) (width 0.2) (layer "F.Cu") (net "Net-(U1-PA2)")))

